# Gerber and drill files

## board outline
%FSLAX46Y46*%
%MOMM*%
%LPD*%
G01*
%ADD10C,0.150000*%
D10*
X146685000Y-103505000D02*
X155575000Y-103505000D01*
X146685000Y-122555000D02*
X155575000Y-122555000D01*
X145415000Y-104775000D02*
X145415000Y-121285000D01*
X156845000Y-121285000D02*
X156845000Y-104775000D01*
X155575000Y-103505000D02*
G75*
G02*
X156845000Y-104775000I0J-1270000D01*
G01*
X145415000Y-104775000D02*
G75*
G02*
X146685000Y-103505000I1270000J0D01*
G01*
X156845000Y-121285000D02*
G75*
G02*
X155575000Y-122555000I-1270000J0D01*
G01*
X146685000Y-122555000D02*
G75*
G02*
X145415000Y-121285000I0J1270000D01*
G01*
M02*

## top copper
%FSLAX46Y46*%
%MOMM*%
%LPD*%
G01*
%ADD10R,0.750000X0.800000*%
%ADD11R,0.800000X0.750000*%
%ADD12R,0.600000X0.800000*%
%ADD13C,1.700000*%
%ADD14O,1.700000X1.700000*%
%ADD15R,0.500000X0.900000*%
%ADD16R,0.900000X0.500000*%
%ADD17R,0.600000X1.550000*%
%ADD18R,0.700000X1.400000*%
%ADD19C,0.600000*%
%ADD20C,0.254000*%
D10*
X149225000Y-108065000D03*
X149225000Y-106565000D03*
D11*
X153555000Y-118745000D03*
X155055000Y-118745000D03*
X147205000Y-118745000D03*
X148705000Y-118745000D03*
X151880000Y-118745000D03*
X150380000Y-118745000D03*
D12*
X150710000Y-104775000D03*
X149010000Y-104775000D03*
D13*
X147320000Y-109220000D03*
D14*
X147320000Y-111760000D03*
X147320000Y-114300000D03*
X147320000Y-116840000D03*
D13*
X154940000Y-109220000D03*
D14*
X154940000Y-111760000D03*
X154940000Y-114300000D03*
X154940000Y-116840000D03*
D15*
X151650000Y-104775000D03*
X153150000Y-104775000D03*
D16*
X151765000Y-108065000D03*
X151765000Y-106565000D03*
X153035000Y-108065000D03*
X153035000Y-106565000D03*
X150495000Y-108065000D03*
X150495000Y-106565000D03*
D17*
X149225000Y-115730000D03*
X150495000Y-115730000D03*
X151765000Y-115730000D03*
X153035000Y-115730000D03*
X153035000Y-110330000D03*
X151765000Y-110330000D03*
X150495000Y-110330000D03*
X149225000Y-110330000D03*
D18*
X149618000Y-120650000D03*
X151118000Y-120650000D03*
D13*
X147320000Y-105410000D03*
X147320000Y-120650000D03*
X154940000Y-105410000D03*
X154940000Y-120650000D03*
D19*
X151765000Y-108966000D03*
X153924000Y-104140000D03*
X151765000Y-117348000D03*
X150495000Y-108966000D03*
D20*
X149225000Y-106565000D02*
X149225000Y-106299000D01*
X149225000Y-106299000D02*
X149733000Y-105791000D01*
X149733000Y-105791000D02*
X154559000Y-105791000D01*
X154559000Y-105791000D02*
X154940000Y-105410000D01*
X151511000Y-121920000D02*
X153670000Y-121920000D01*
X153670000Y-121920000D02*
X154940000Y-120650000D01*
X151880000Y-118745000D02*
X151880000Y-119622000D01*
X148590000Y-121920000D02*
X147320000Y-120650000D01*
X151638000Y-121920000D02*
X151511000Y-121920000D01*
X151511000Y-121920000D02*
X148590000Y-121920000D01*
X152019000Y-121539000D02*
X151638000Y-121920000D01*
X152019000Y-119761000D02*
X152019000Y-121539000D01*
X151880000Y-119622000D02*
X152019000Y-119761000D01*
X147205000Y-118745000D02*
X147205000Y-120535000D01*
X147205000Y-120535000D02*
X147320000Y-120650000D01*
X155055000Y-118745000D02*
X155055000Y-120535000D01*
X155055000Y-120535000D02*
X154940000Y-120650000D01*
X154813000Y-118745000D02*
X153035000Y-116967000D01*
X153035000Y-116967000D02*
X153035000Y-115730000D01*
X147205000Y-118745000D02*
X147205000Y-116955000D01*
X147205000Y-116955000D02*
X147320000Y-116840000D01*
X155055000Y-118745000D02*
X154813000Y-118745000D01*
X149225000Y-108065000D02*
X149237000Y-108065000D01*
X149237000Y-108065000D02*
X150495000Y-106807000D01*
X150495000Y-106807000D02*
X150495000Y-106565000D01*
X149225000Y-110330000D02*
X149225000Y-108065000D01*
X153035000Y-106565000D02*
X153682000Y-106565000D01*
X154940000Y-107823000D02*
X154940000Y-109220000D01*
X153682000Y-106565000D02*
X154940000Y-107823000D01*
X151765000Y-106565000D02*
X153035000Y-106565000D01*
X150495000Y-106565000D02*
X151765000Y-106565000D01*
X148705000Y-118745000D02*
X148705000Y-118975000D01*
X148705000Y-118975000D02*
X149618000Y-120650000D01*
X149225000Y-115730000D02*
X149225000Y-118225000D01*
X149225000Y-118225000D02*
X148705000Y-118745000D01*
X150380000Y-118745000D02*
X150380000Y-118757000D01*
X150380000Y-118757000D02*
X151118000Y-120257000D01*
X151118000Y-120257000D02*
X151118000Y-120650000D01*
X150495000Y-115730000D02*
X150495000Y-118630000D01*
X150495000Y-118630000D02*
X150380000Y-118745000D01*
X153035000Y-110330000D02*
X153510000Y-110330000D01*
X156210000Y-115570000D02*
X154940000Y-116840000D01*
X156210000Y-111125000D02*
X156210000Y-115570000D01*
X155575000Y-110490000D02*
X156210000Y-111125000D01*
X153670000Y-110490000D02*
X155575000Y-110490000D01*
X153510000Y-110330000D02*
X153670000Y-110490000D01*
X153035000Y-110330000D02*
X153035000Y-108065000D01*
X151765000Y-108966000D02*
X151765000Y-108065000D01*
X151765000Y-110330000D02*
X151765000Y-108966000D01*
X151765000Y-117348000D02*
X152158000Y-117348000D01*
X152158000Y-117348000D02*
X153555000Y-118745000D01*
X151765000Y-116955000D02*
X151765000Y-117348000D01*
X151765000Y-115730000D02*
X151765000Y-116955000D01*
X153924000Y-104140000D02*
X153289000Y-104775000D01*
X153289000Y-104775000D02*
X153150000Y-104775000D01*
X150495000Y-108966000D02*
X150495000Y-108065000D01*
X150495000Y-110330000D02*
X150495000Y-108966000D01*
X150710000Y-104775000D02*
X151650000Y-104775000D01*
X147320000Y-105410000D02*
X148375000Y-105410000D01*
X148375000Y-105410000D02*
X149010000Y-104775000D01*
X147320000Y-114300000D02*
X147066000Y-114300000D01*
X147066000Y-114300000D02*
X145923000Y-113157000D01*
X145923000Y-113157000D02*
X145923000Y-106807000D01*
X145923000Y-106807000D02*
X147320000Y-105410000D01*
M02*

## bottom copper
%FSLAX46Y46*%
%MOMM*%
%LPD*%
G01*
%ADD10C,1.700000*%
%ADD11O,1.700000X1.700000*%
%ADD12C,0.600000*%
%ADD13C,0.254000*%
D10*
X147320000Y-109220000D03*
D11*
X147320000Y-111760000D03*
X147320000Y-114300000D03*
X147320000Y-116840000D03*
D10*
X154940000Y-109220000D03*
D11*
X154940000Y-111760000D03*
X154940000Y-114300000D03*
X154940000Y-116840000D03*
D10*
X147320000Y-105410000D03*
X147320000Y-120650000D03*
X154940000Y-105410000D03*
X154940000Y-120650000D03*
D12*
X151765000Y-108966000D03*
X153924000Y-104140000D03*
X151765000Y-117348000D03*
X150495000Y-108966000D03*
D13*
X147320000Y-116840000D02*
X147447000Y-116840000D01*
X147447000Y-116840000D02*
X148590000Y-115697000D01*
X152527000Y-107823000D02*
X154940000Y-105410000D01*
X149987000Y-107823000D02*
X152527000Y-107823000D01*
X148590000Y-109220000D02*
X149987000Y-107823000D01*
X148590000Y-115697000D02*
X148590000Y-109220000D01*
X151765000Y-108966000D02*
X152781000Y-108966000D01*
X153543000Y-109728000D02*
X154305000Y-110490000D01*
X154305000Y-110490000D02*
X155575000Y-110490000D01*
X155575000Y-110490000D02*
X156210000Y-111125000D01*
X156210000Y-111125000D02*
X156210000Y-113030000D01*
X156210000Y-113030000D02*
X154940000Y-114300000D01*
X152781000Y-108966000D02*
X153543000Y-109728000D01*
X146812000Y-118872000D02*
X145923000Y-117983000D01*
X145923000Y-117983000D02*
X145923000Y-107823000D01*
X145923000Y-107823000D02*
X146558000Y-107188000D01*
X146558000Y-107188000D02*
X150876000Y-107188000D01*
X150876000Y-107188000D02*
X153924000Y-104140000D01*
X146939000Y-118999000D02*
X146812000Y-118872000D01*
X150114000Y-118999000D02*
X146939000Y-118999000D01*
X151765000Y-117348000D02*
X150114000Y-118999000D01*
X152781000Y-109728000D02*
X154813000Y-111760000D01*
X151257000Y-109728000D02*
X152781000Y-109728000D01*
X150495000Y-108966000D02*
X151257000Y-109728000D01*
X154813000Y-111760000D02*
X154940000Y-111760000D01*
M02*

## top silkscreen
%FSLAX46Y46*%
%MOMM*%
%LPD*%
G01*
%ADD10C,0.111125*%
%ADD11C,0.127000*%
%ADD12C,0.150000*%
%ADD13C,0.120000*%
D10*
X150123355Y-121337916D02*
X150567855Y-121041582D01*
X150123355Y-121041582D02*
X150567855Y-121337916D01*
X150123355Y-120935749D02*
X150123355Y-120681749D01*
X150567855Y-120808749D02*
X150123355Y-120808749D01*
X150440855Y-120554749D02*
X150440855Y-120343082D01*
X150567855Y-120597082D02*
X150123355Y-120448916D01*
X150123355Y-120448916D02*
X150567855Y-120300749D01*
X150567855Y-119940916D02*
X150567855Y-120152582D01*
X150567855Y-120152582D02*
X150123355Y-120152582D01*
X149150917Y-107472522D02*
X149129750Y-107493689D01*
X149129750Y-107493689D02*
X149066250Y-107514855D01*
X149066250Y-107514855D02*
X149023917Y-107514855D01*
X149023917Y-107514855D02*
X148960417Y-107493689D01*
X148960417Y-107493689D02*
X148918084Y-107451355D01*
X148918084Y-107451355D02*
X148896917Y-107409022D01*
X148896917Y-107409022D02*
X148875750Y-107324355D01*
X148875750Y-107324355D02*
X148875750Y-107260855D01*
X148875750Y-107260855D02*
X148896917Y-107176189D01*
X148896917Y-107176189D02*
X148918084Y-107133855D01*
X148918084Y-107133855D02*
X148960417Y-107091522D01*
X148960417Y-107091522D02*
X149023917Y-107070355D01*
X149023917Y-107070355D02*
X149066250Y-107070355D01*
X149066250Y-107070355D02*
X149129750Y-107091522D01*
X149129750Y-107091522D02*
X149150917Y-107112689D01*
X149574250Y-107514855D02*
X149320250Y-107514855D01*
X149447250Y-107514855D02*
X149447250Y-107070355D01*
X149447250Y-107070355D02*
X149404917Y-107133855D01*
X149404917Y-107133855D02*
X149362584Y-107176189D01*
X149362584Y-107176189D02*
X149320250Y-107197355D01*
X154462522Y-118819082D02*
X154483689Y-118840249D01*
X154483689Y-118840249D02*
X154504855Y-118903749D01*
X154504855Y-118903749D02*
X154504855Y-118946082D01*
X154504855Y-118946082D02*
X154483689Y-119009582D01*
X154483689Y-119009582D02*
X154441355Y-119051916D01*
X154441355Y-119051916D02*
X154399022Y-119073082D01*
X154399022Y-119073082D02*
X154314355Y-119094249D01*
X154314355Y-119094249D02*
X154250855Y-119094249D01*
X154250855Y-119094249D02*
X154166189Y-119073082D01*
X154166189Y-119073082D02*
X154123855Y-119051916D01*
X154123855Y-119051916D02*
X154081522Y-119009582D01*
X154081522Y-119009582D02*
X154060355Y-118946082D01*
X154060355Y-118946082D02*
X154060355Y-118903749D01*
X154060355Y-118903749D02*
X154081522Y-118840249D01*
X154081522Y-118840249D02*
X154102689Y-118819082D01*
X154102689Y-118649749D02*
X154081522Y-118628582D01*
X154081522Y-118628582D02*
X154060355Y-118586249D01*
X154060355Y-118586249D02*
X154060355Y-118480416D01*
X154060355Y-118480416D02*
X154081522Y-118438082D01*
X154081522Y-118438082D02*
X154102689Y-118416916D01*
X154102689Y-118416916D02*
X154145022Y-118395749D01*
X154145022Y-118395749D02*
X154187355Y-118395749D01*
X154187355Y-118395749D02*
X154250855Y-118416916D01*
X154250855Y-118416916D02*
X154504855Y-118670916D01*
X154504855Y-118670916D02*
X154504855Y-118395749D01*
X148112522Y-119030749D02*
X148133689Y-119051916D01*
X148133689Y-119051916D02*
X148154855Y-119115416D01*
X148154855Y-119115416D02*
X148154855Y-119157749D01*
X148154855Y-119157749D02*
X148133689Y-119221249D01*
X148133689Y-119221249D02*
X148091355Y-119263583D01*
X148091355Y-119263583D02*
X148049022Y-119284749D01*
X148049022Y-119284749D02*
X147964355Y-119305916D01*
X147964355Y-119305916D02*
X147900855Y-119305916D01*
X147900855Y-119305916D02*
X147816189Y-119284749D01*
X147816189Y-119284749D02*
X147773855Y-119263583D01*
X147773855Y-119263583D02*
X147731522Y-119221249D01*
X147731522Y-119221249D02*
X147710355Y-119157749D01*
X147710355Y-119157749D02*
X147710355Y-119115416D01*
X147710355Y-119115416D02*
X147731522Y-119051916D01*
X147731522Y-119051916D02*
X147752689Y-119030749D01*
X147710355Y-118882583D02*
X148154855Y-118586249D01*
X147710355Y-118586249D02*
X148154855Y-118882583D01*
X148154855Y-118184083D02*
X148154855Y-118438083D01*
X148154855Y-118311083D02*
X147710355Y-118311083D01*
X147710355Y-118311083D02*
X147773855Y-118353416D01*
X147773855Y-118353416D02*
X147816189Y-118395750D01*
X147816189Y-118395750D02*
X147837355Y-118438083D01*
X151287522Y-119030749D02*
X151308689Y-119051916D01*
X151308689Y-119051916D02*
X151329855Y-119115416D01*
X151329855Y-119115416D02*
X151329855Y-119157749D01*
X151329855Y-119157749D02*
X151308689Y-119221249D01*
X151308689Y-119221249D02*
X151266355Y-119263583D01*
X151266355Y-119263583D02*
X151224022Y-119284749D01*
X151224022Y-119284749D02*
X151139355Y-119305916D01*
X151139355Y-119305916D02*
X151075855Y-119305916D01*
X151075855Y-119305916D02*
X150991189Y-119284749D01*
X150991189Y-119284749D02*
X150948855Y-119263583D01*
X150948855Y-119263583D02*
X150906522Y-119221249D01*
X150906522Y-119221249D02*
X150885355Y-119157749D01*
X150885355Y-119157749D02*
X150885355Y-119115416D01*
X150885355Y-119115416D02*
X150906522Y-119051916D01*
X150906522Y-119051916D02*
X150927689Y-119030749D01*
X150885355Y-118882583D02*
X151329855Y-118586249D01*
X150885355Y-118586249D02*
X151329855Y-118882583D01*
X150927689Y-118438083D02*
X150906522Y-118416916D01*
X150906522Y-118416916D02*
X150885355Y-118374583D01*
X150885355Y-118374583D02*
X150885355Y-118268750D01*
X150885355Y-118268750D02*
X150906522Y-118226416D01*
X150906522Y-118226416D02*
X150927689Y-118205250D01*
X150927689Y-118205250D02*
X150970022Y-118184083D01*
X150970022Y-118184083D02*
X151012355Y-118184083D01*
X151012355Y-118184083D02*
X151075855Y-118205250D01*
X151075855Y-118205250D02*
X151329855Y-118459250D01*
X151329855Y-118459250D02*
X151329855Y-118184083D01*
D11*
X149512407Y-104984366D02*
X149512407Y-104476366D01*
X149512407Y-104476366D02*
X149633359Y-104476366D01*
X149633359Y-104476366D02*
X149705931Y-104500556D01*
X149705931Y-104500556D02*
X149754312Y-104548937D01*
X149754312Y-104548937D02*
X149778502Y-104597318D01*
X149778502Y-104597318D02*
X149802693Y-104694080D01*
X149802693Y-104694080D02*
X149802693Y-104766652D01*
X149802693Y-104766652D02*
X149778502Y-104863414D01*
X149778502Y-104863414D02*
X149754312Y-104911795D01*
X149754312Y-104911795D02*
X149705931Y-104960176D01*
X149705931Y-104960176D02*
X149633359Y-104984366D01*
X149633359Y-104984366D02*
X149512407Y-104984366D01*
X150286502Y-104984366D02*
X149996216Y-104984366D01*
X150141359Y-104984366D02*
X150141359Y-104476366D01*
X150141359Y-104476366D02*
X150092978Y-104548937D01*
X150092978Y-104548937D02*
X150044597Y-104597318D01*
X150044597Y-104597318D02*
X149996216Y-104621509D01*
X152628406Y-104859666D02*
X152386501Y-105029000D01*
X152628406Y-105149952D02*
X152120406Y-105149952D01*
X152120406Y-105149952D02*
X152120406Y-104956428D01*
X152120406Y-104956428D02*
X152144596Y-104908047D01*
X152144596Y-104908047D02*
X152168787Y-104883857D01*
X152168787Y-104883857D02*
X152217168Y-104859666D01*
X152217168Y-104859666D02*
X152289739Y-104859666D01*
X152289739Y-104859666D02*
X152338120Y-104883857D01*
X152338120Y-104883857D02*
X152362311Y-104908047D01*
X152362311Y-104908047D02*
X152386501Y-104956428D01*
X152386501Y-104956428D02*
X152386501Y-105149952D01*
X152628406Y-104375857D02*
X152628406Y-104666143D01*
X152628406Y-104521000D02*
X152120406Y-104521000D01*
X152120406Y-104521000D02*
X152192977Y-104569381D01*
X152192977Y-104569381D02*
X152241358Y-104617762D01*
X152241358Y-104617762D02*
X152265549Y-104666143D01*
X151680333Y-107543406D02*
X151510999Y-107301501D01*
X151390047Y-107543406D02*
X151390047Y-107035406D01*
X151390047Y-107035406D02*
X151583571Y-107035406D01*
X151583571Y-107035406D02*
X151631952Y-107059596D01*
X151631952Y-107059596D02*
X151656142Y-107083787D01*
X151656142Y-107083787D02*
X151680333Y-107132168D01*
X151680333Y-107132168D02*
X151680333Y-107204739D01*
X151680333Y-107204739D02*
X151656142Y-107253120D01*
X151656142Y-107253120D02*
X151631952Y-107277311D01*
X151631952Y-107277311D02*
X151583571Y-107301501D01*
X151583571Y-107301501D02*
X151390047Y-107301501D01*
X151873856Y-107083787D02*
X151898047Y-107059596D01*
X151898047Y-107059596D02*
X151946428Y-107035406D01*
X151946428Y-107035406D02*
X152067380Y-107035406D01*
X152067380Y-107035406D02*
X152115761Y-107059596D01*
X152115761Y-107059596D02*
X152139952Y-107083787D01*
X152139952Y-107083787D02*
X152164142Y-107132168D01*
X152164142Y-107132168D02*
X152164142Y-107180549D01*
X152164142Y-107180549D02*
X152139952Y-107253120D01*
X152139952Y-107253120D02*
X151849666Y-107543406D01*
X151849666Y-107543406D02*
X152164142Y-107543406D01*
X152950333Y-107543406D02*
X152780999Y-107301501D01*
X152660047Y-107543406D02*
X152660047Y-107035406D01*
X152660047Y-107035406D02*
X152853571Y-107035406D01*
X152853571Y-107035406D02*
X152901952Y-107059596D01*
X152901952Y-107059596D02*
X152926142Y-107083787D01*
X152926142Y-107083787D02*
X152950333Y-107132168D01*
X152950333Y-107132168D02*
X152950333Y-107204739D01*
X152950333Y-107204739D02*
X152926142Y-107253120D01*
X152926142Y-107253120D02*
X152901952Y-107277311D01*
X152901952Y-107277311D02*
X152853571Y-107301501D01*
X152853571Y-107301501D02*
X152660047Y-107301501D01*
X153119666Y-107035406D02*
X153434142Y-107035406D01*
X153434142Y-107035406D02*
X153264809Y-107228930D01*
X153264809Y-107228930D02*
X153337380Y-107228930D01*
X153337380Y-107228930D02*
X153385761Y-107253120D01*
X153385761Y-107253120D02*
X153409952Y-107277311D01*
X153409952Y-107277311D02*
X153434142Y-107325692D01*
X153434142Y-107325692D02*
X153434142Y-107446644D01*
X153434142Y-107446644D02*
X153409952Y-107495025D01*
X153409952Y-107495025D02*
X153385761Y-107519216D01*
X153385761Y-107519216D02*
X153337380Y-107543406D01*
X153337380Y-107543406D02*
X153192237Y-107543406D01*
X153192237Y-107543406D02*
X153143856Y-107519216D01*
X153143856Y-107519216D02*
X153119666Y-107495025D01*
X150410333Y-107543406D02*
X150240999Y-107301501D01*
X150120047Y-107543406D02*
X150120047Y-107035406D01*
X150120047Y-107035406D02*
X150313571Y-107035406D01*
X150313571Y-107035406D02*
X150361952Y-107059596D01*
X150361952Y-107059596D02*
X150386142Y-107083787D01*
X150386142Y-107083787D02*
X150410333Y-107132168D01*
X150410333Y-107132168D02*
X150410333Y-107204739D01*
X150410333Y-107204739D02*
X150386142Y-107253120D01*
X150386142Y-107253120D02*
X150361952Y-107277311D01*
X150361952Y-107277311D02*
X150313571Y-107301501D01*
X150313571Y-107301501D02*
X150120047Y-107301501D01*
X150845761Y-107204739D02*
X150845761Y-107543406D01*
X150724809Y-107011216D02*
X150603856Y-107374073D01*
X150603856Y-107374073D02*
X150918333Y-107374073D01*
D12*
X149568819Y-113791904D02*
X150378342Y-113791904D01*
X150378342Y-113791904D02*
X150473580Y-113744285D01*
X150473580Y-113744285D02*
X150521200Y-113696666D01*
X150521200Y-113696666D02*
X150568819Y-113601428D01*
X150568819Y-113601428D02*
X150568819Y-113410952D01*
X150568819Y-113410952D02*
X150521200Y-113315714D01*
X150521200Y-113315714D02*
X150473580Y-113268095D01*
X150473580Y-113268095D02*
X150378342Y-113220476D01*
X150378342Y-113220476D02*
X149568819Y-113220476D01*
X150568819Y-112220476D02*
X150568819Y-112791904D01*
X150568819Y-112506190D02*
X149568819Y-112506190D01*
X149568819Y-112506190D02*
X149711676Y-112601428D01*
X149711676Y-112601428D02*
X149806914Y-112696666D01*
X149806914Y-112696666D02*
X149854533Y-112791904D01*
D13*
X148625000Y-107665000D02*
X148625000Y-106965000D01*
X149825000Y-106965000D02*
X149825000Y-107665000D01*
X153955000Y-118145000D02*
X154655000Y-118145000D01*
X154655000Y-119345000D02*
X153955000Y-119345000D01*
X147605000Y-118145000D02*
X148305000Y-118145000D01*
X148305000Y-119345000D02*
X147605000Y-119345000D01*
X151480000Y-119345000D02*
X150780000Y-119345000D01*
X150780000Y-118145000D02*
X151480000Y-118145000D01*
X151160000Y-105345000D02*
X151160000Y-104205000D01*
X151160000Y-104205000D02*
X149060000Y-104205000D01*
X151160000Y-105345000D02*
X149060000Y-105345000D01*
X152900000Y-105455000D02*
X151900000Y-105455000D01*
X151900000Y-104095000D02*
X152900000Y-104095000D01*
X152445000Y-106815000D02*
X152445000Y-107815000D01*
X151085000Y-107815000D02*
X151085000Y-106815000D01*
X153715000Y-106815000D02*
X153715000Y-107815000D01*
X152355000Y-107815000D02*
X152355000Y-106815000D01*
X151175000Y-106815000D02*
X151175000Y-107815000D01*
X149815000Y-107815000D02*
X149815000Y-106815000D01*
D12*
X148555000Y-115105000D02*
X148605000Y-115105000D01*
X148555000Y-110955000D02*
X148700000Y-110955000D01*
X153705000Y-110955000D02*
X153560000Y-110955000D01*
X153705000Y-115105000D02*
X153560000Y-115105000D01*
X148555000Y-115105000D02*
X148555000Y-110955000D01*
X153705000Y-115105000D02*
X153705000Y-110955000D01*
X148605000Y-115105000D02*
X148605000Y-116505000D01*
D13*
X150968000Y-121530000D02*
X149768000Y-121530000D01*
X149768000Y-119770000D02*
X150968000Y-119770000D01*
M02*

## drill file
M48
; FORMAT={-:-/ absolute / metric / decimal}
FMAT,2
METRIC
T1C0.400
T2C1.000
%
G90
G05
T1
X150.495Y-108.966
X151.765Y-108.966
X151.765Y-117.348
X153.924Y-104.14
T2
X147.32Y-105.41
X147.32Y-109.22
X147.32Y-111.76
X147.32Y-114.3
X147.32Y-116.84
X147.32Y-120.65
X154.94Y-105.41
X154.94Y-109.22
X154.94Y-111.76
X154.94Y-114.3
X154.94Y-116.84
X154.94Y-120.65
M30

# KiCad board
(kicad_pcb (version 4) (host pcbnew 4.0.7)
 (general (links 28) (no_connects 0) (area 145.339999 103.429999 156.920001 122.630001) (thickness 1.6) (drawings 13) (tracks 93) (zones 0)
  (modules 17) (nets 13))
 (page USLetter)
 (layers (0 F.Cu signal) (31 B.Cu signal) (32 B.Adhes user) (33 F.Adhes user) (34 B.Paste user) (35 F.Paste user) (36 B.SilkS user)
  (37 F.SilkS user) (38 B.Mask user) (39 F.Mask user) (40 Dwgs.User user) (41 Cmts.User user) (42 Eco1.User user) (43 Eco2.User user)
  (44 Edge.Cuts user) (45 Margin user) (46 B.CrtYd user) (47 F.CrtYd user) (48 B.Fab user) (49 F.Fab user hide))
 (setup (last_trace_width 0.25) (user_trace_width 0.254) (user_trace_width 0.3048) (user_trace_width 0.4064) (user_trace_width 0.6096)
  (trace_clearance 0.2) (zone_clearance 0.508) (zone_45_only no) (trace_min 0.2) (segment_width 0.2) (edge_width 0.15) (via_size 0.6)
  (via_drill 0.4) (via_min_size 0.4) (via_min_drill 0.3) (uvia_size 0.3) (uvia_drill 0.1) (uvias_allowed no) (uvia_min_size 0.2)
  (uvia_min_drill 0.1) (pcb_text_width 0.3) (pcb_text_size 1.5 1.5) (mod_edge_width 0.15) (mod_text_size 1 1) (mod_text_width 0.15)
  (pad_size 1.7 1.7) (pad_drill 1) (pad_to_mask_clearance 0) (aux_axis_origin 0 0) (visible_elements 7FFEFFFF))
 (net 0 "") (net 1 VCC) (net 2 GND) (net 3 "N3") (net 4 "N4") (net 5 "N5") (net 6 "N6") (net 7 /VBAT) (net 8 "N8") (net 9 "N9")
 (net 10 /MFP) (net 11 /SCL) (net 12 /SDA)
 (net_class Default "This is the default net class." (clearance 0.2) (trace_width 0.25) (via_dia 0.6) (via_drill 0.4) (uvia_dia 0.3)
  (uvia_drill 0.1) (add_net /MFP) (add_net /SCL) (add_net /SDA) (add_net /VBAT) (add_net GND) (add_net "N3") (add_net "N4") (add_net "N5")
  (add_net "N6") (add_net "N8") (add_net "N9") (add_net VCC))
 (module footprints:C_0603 (layer F.Cu) (at 149.225 107.315 270)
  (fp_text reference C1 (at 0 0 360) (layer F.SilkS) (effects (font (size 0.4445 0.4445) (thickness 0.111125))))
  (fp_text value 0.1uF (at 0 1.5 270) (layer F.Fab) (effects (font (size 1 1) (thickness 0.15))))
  (fp_line (start 0.35 0.6) (end -0.35 0.6) (layer F.SilkS) (width 0.12))
  (fp_line (start -0.35 -0.6) (end 0.35 -0.6) (layer F.SilkS) (width 0.12))
  (pad 2 smd rect (at 0.75 0 270) (size 0.8 0.75) (layers F.Cu F.Paste F.Mask) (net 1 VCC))
  (pad 1 smd rect (at -0.75 0 270) (size 0.8 0.75) (layers F.Cu F.Paste F.Mask) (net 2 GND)))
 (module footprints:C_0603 (layer F.Cu) (at 154.305 118.745 180)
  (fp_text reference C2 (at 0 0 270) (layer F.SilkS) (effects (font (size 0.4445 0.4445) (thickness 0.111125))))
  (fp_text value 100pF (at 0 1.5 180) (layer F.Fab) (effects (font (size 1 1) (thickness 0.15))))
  (fp_line (start 0.35 0.6) (end -0.35 0.6) (layer F.SilkS) (width 0.12))
  (fp_line (start -0.35 -0.6) (end 0.35 -0.6) (layer F.SilkS) (width 0.12))
  (pad 2 smd rect (at 0.75 0 180) (size 0.8 0.75) (layers F.Cu F.Paste F.Mask) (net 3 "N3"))
  (pad 1 smd rect (at -0.75 0 180) (size 0.8 0.75) (layers F.Cu F.Paste F.Mask) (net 2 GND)))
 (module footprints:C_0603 (layer F.Cu) (at 147.955 118.745 180)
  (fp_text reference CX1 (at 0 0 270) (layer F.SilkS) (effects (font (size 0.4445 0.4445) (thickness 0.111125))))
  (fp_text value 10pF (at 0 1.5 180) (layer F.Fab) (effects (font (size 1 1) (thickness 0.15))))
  (fp_line (start 0.35 0.6) (end -0.35 0.6) (layer F.SilkS) (width 0.12))
  (fp_line (start -0.35 -0.6) (end 0.35 -0.6) (layer F.SilkS) (width 0.12))
  (pad 2 smd rect (at 0.75 0 180) (size 0.8 0.75) (layers F.Cu F.Paste F.Mask) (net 2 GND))
  (pad 1 smd rect (at -0.75 0 180) (size 0.8 0.75) (layers F.Cu F.Paste F.Mask) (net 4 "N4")))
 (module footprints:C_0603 (layer F.Cu) (at 151.13 118.745)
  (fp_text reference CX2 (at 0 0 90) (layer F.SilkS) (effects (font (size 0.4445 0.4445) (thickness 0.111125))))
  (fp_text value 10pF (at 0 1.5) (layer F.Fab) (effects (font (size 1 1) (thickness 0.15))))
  (fp_line (start 0.35 0.6) (end -0.35 0.6) (layer F.SilkS) (width 0.12))
  (fp_line (start -0.35 -0.6) (end 0.35 -0.6) (layer F.SilkS) (width 0.12))
  (pad 2 smd rect (at 0.75 0) (size 0.8 0.75) (layers F.Cu F.Paste F.Mask) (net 2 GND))
  (pad 1 smd rect (at -0.75 0) (size 0.8 0.75) (layers F.Cu F.Paste F.Mask) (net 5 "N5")))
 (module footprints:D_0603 (layer F.Cu) (at 149.86 104.775 180)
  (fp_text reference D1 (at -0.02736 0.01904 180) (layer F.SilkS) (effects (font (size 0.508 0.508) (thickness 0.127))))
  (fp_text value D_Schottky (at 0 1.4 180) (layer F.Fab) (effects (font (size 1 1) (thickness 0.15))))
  (fp_line (start -1.3 -0.57) (end -1.3 0.57) (layer F.SilkS) (width 0.12))
  (fp_line (start -1.3 0.57) (end 0.8 0.57) (layer F.SilkS) (width 0.12))
  (fp_line (start -1.3 -0.57) (end 0.8 -0.57) (layer F.SilkS) (width 0.12))
  (pad 1 smd rect (at -0.85 0 180) (size 0.6 0.8) (layers F.Cu F.Paste F.Mask) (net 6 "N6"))
  (pad 2 smd rect (at 0.85 0 180) (size 0.6 0.8) (layers F.Cu F.Paste F.Mask) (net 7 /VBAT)))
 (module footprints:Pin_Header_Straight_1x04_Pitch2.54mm (layer F.Cu) (at 147.32 109.22)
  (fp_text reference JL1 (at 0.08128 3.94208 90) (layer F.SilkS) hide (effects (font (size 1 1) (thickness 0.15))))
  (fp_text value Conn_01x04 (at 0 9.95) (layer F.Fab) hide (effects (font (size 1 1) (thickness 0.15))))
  (pad 1 thru_hole circle (at 0 0) (size 1.7 1.7) (drill 1) (layers *.Cu *.Mask) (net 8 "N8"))
  (pad 2 thru_hole oval (at 0 2.54) (size 1.7 1.7) (drill 1) (layers *.Cu *.Mask) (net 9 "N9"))
  (pad 3 thru_hole oval (at 0 5.08) (size 1.7 1.7) (drill 1) (layers *.Cu *.Mask) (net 7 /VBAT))
  (pad 4 thru_hole oval (at 0 7.62) (size 1.7 1.7) (drill 1) (layers *.Cu *.Mask) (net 2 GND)))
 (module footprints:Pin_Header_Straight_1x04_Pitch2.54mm (layer F.Cu) (at 154.94 109.22)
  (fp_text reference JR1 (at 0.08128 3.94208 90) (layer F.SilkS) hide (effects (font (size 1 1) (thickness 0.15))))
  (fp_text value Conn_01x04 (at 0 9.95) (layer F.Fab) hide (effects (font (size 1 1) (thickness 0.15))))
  (pad 1 thru_hole circle (at 0 0) (size 1.7 1.7) (drill 1) (layers *.Cu *.Mask) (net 1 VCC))
  (pad 2 thru_hole oval (at 0 2.54) (size 1.7 1.7) (drill 1) (layers *.Cu *.Mask) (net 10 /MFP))
  (pad 3 thru_hole oval (at 0 5.08) (size 1.7 1.7) (drill 1) (layers *.Cu *.Mask) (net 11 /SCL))
  (pad 4 thru_hole oval (at 0 7.62) (size 1.7 1.7) (drill 1) (layers *.Cu *.Mask) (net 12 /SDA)))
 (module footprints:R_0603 (layer F.Cu) (at 152.4 104.775)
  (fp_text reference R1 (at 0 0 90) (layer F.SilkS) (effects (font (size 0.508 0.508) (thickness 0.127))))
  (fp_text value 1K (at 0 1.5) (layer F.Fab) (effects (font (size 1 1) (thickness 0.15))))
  (fp_line (start 0.5 0.68) (end -0.5 0.68) (layer F.SilkS) (width 0.12))
  (fp_line (start -0.5 -0.68) (end 0.5 -0.68) (layer F.SilkS) (width 0.12))
  (pad 1 smd rect (at -0.75 0) (size 0.5 0.9) (layers F.Cu F.Paste F.Mask) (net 6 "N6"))
  (pad 2 smd rect (at 0.75 0) (size 0.5 0.9) (layers F.Cu F.Paste F.Mask) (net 3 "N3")))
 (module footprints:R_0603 (layer F.Cu) (at 151.765 107.315 90)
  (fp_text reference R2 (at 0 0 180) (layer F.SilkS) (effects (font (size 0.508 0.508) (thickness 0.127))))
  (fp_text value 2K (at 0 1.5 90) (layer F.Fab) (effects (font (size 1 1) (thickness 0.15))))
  (fp_line (start 0.5 0.68) (end -0.5 0.68) (layer F.SilkS) (width 0.12))
  (fp_line (start -0.5 -0.68) (end 0.5 -0.68) (layer F.SilkS) (width 0.12))
  (pad 1 smd rect (at -0.75 0 90) (size 0.5 0.9) (layers F.Cu F.Paste F.Mask) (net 11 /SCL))
  (pad 2 smd rect (at 0.75 0 90) (size 0.5 0.9) (layers F.Cu F.Paste F.Mask) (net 1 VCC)))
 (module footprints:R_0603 (layer F.Cu) (at 153.035 107.315 90)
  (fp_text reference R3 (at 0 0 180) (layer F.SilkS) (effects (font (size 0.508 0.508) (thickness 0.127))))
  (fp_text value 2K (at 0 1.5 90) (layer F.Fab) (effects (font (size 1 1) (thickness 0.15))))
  (fp_line (start 0.5 0.68) (end -0.5 0.68) (layer F.SilkS) (width 0.12))
  (fp_line (start -0.5 -0.68) (end 0.5 -0.68) (layer F.SilkS) (width 0.12))
  (pad 1 smd rect (at -0.75 0 90) (size 0.5 0.9) (layers F.Cu F.Paste F.Mask) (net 12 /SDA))
  (pad 2 smd rect (at 0.75 0 90) (size 0.5 0.9) (layers F.Cu F.Paste F.Mask) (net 1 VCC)))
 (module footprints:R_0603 (layer F.Cu) (at 150.495 107.315 90)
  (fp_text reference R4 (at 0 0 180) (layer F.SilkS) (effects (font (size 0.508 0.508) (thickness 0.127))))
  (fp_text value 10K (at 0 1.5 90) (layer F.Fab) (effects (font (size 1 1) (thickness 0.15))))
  (fp_line (start 0.5 0.68) (end -0.5 0.68) (layer F.SilkS) (width 0.12))
  (fp_line (start -0.5 -0.68) (end 0.5 -0.68) (layer F.SilkS) (width 0.12))
  (pad 1 smd rect (at -0.75 0 90) (size 0.5 0.9) (layers F.Cu F.Paste F.Mask) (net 10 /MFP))
  (pad 2 smd rect (at 0.75 0 90) (size 0.5 0.9) (layers F.Cu F.Paste F.Mask) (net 1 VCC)))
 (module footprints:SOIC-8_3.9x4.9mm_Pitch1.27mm (layer F.Cu) (at 151.13 113.03 90)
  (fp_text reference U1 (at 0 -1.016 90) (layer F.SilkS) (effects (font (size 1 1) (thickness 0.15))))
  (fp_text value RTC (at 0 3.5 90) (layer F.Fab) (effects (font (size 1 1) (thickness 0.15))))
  (fp_line (start -2.075 -2.575) (end -2.075 -2.525) (layer F.SilkS) (width 0.15))
  (fp_line (start 2.075 -2.575) (end 2.075 -2.43) (layer F.SilkS) (width 0.15))
  (fp_line (start 2.075 2.575) (end 2.075 2.43) (layer F.SilkS) (width 0.15))
  (fp_line (start -2.075 2.575) (end -2.075 2.43) (layer F.SilkS) (width 0.15))
  (fp_line (start -2.075 -2.575) (end 2.075 -2.575) (layer F.SilkS) (width 0.15))
  (fp_line (start -2.075 2.575) (end 2.075 2.575) (layer F.SilkS) (width 0.15))
  (fp_line (start -2.075 -2.525) (end -3.475 -2.525) (layer F.SilkS) (width 0.15))
  (pad 1 smd rect (at -2.7 -1.905 90) (size 1.55 0.6) (layers F.Cu F.Paste F.Mask) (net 4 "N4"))
  (pad 2 smd rect (at -2.7 -0.635 90) (size 1.55 0.6) (layers F.Cu F.Paste F.Mask) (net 5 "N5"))
  (pad 3 smd rect (at -2.7 0.635 90) (size 1.55 0.6) (layers F.Cu F.Paste F.Mask) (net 3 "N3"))
  (pad 4 smd rect (at -2.7 1.905 90) (size 1.55 0.6) (layers F.Cu F.Paste F.Mask) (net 2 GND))
  (pad 5 smd rect (at 2.7 1.905 90) (size 1.55 0.6) (layers F.Cu F.Paste F.Mask) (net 12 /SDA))
  (pad 6 smd rect (at 2.7 0.635 90) (size 1.55 0.6) (layers F.Cu F.Paste F.Mask) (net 11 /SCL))
  (pad 7 smd rect (at 2.7 -0.635 90) (size 1.55 0.6) (layers F.Cu F.Paste F.Mask) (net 10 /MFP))
  (pad 8 smd rect (at 2.7 -1.905 90) (size 1.55 0.6) (layers F.Cu F.Paste F.Mask) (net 1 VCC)))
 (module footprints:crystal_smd (layer F.Cu) (at 150.368 120.65)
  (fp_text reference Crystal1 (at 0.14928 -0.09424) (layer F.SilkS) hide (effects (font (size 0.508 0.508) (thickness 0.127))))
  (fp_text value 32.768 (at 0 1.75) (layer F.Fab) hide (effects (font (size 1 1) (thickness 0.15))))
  (fp_line (start 0.6 0.88) (end -0.6 0.88) (layer F.SilkS) (width 0.12))
  (fp_line (start -0.6 -0.88) (end 0.6 -0.88) (layer F.SilkS) (width 0.12))
  (pad 1 smd rect (at -0.75 0) (size 0.7 1.4) (layers F.Cu F.Paste F.Mask) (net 4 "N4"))
  (pad 2 smd rect (at 0.75 0) (size 0.7 1.4) (layers F.Cu F.Paste F.Mask) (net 5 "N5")))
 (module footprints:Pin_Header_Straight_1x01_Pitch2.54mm (layer F.Cu) (at 147.32 105.41)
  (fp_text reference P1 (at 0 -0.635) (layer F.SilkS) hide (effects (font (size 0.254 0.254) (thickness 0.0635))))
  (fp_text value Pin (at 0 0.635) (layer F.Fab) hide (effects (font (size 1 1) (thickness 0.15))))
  (pad 1 thru_hole circle (at 0 0) (size 1.7 1.7) (drill 1) (layers *.Cu *.Mask) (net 7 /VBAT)))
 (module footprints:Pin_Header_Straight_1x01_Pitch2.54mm (layer F.Cu) (at 147.32 120.65)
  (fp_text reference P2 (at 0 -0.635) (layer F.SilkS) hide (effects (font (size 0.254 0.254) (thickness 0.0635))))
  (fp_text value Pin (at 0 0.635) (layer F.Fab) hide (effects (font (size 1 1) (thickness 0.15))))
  (pad 1 thru_hole circle (at 0 0) (size 1.7 1.7) (drill 1) (layers *.Cu *.Mask) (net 2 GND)))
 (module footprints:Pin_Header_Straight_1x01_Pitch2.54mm (layer F.Cu) (at 154.94 105.41)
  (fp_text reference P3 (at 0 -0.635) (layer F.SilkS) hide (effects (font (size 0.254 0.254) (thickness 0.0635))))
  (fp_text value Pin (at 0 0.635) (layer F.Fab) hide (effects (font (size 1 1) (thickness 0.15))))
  (pad 1 thru_hole circle (at 0 0) (size 1.7 1.7) (drill 1) (layers *.Cu *.Mask) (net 2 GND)))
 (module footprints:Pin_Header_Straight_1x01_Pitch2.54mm (layer F.Cu) (at 154.94 120.65)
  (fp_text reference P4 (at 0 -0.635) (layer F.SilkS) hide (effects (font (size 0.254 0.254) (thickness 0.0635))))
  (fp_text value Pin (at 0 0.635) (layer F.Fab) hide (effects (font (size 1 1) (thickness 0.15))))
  (pad 1 thru_hole circle (at 0 0) (size 1.7 1.7) (drill 1) (layers *.Cu *.Mask) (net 2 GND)))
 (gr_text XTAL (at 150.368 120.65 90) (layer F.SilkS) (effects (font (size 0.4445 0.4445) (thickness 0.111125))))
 (gr_line (start 146.685 103.505) (end 155.575 103.505) (angle 90) (layer Edge.Cuts) (width 0.15))
 (gr_line (start 146.685 122.555) (end 155.575 122.555) (angle 90) (layer Edge.Cuts) (width 0.15))
 (gr_line (start 145.415 104.775) (end 145.415 121.285) (angle 90) (layer Edge.Cuts) (width 0.15))
 (gr_line (start 156.845 121.285) (end 156.845 104.775) (angle 90) (layer Edge.Cuts) (width 0.15))
 (gr_arc (start 155.575 104.775) (end 155.575 103.505) (angle 90) (layer Edge.Cuts) (width 0.15))
 (gr_arc (start 146.685 104.775) (end 145.415 104.775) (angle 90) (layer Edge.Cuts) (width 0.15))
 (gr_arc (start 155.575 121.285) (end 156.845 121.285) (angle 90) (layer Edge.Cuts) (width 0.15))
 (gr_arc (start 146.685 121.285) (end 146.685 122.555) (angle 90) (layer Edge.Cuts) (width 0.15))
 (segment (start 147.32 116.84) (end 147.447 116.84) (width 0.254) (layer B.Cu) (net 2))
 (segment (start 147.447 116.84) (end 148.59 115.697) (width 0.254) (layer B.Cu) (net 2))
 (segment (start 152.527 107.823) (end 154.94 105.41) (width 0.254) (layer B.Cu) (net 2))
 (segment (start 149.987 107.823) (end 152.527 107.823) (width 0.254) (layer B.Cu) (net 2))
 (segment (start 148.59 109.22) (end 149.987 107.823) (width 0.254) (layer B.Cu) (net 2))
 (segment (start 148.59 115.697) (end 148.59 109.22) (width 0.254) (layer B.Cu) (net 2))
 (segment (start 149.225 106.565) (end 149.225 106.299) (width 0.254) (layer F.Cu) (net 2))
 (segment (start 149.225 106.299) (end 149.733 105.791) (width 0.254) (layer F.Cu) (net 2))
 (segment (start 149.733 105.791) (end 154.559 105.791) (width 0.254) (layer F.Cu) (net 2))
 (segment (start 154.559 105.791) (end 154.94 105.41) (width 0.254) (layer F.Cu) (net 2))
 (segment (start 151.511 121.92) (end 153.67 121.92) (width 0.254) (layer F.Cu) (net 2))
 (segment (start 153.67 121.92) (end 154.94 120.65) (width 0.254) (layer F.Cu) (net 2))
 (segment (start 151.88 118.745) (end 151.88 119.622) (width 0.254) (layer F.Cu) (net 2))
 (segment (start 148.59 121.92) (end 147.32 120.65) (width 0.254) (layer F.Cu) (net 2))
 (segment (start 151.638 121.92) (end 151.511 121.92) (width 0.254) (layer F.Cu) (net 2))
 (segment (start 151.511 121.92) (end 148.59 121.92) (width 0.254) (layer F.Cu) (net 2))
 (segment (start 152.019 121.539) (end 151.638 121.92) (width 0.254) (layer F.Cu) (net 2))
 (segment (start 152.019 119.761) (end 152.019 121.539) (width 0.254) (layer F.Cu) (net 2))
 (segment (start 151.88 119.622) (end 152.019 119.761) (width 0.254) (layer F.Cu) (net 2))
 (segment (start 147.205 118.745) (end 147.205 120.535) (width 0.254) (layer F.Cu) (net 2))
 (segment (start 147.205 120.535) (end 147.32 120.65) (width 0.254) (layer F.Cu) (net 2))
 (segment (start 155.055 118.745) (end 155.055 120.535) (width 0.254) (layer F.Cu) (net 2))
 (segment (start 155.055 120.535) (end 154.94 120.65) (width 0.254) (layer F.Cu) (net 2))
 (segment (start 154.813 118.745) (end 153.035 116.967) (width 0.254) (layer F.Cu) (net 2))
 (segment (start 153.035 116.967) (end 153.035 115.73) (width 0.254) (layer F.Cu) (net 2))
 (segment (start 147.205 118.745) (end 147.205 116.955) (width 0.254) (layer F.Cu) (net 2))
 (segment (start 147.205 116.955) (end 147.32 116.84) (width 0.254) (layer F.Cu) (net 2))
 (segment (start 155.055 118.745) (end 154.813 118.745) (width 0.254) (layer F.Cu) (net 2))
 (segment (start 149.225 108.065) (end 149.237 108.065) (width 0.254) (layer F.Cu) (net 1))
 (segment (start 149.237 108.065) (end 150.495 106.807) (width 0.254) (layer F.Cu) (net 1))
 (segment (start 150.495 106.807) (end 150.495 106.565) (width 0.254) (layer F.Cu) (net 1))
 (segment (start 149.225 110.33) (end 149.225 108.065) (width 0.254) (layer F.Cu) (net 1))
 (segment (start 153.035 106.565) (end 153.682 106.565) (width 0.254) (layer F.Cu) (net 1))
 (segment (start 154.94 107.823) (end 154.94 109.22) (width 0.254) (layer F.Cu) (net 1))
 (segment (start 153.682 106.565) (end 154.94 107.823) (width 0.254) (layer F.Cu) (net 1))
 (segment (start 151.765 106.565) (end 153.035 106.565) (width 0.254) (layer F.Cu) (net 1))
 (segment (start 150.495 106.565) (end 151.765 106.565) (width 0.254) (layer F.Cu) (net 1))
 (segment (start 148.705 118.745) (end 148.705 118.975) (width 0.254) (layer F.Cu) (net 4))
 (segment (start 148.705 118.975) (end 149.618 120.65) (width 0.254) (layer F.Cu) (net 4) (status 20))
 (segment (start 149.225 115.73) (end 149.225 118.225) (width 0.254) (layer F.Cu) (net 4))
 (segment (start 149.225 118.225) (end 148.705 118.745) (width 0.254) (layer F.Cu) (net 4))
 (segment (start 150.38 118.745) (end 150.38 118.757) (width 0.254) (layer F.Cu) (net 5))
 (segment (start 150.38 118.757) (end 151.118 120.257) (width 0.254) (layer F.Cu) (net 5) (status 20))
 (segment (start 151.118 120.257) (end 151.118 120.65) (width 0.254) (layer F.Cu) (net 5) (status 30))
 (segment (start 150.495 115.73) (end 150.495 118.63) (width 0.254) (layer F.Cu) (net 5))
 (segment (start 150.495 118.63) (end 150.38 118.745) (width 0.254) (layer F.Cu) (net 5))
 (segment (start 153.035 110.33) (end 153.51 110.33) (width 0.254) (layer F.Cu) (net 12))
 (segment (start 156.21 115.57) (end 154.94 116.84) (width 0.254) (layer F.Cu) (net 12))
 (segment (start 156.21 111.125) (end 156.21 115.57) (width 0.254) (layer F.Cu) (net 12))
 (segment (start 155.575 110.49) (end 156.21 111.125) (width 0.254) (layer F.Cu) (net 12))
 (segment (start 153.67 110.49) (end 155.575 110.49) (width 0.254) (layer F.Cu) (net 12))
 (segment (start 153.51 110.33) (end 153.67 110.49) (width 0.254) (layer F.Cu) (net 12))
 (segment (start 153.035 110.33) (end 153.035 108.065) (width 0.254) (layer F.Cu) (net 12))
 (segment (start 151.765 108.966) (end 152.781 108.966) (width 0.254) (layer B.Cu) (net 11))
 (segment (start 153.543 109.728) (end 154.305 110.49) (width 0.254) (layer B.Cu) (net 11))
 (segment (start 154.305 110.49) (end 155.575 110.49) (width 0.254) (layer B.Cu) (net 11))
 (segment (start 155.575 110.49) (end 156.21 111.125) (width 0.254) (layer B.Cu) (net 11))
 (segment (start 156.21 111.125) (end 156.21 113.03) (width 0.254) (layer B.Cu) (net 11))
 (segment (start 156.21 113.03) (end 154.94 114.3) (width 0.254) (layer B.Cu) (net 11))
 (via (at 151.765 108.966) (size 0.6) (drill 0.4) (layers F.Cu B.Cu) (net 11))
 (segment (start 152.781 108.966) (end 153.543 109.728) (width 0.254) (layer B.Cu) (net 11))
 (segment (start 151.765 108.966) (end 151.765 108.065) (width 0.254) (layer F.Cu) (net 11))
 (segment (start 151.765 110.33) (end 151.765 108.966) (width 0.254) (layer F.Cu) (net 11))
 (segment (start 151.765 117.348) (end 152.158 117.348) (width 0.254) (layer F.Cu) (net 3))
 (segment (start 152.158 117.348) (end 153.555 118.745) (width 0.254) (layer F.Cu) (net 3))
 (segment (start 151.765 116.955) (end 151.765 117.348) (width 0.254) (layer F.Cu) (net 3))
 (segment (start 151.765 115.73) (end 151.765 116.955) (width 0.254) (layer F.Cu) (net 3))
 (segment (start 146.812 118.872) (end 145.923 117.983) (width 0.254) (layer B.Cu) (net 3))
 (segment (start 145.923 117.983) (end 145.923 107.823) (width 0.254) (layer B.Cu) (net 3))
 (segment (start 145.923 107.823) (end 146.558 107.188) (width 0.254) (layer B.Cu) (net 3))
 (segment (start 146.558 107.188) (end 150.876 107.188) (width 0.254) (layer B.Cu) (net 3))
 (segment (start 150.876 107.188) (end 153.924 104.14) (width 0.254) (layer B.Cu) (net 3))
 (via (at 153.924 104.14) (size 0.6) (drill 0.4) (layers F.Cu B.Cu) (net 3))
 (segment (start 153.924 104.14) (end 153.289 104.775) (width 0.254) (layer F.Cu) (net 3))
 (segment (start 146.939 118.999) (end 146.812 118.872) (width 0.254) (layer B.Cu) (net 3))
 (segment (start 150.114 118.999) (end 146.939 118.999) (width 0.254) (layer B.Cu) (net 3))
 (segment (start 151.765 117.348) (end 150.114 118.999) (width 0.254) (layer B.Cu) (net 3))
 (via (at 151.765 117.348) (size 0.6) (drill 0.4) (layers F.Cu B.Cu) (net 3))
 (segment (start 153.289 104.775) (end 153.15 104.775) (width 0.254) (layer F.Cu) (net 3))
 (segment (start 150.495 108.966) (end 150.495 108.065) (width 0.254) (layer F.Cu) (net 10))
 (segment (start 150.495 110.33) (end 150.495 108.966) (width 0.254) (layer F.Cu) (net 10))
 (segment (start 152.781 109.728) (end 154.813 111.76) (width 0.254) (layer B.Cu) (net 10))
 (segment (start 151.257 109.728) (end 152.781 109.728) (width 0.254) (layer B.Cu) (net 10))
 (segment (start 150.495 108.966) (end 151.257 109.728) (width 0.254) (layer B.Cu) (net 10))
 (via (at 150.495 108.966) (size 0.6) (drill 0.4) (layers F.Cu B.Cu) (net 10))
 (segment (start 154.813 111.76) (end 154.94 111.76) (width 0.254) (layer B.Cu) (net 10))
 (segment (start 150.71 104.775) (end 151.65 104.775) (width 0.254) (layer F.Cu) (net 6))
 (segment (start 147.32 105.41) (end 148.375 105.41) (width 0.254) (layer F.Cu) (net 7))
 (segment (start 148.375 105.41) (end 149.01 104.775) (width 0.254) (layer F.Cu) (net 7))
 (segment (start 147.32 114.3) (end 147.066 114.3) (width 0.254) (layer F.Cu) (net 7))
 (segment (start 147.066 114.3) (end 145.923 113.157) (width 0.254) (layer F.Cu) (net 7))
 (segment (start 145.923 113.157) (end 145.923 106.807) (width 0.254) (layer F.Cu) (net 7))
 (segment (start 145.923 106.807) (end 147.32 105.41) (width 0.254) (layer F.Cu) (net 7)))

